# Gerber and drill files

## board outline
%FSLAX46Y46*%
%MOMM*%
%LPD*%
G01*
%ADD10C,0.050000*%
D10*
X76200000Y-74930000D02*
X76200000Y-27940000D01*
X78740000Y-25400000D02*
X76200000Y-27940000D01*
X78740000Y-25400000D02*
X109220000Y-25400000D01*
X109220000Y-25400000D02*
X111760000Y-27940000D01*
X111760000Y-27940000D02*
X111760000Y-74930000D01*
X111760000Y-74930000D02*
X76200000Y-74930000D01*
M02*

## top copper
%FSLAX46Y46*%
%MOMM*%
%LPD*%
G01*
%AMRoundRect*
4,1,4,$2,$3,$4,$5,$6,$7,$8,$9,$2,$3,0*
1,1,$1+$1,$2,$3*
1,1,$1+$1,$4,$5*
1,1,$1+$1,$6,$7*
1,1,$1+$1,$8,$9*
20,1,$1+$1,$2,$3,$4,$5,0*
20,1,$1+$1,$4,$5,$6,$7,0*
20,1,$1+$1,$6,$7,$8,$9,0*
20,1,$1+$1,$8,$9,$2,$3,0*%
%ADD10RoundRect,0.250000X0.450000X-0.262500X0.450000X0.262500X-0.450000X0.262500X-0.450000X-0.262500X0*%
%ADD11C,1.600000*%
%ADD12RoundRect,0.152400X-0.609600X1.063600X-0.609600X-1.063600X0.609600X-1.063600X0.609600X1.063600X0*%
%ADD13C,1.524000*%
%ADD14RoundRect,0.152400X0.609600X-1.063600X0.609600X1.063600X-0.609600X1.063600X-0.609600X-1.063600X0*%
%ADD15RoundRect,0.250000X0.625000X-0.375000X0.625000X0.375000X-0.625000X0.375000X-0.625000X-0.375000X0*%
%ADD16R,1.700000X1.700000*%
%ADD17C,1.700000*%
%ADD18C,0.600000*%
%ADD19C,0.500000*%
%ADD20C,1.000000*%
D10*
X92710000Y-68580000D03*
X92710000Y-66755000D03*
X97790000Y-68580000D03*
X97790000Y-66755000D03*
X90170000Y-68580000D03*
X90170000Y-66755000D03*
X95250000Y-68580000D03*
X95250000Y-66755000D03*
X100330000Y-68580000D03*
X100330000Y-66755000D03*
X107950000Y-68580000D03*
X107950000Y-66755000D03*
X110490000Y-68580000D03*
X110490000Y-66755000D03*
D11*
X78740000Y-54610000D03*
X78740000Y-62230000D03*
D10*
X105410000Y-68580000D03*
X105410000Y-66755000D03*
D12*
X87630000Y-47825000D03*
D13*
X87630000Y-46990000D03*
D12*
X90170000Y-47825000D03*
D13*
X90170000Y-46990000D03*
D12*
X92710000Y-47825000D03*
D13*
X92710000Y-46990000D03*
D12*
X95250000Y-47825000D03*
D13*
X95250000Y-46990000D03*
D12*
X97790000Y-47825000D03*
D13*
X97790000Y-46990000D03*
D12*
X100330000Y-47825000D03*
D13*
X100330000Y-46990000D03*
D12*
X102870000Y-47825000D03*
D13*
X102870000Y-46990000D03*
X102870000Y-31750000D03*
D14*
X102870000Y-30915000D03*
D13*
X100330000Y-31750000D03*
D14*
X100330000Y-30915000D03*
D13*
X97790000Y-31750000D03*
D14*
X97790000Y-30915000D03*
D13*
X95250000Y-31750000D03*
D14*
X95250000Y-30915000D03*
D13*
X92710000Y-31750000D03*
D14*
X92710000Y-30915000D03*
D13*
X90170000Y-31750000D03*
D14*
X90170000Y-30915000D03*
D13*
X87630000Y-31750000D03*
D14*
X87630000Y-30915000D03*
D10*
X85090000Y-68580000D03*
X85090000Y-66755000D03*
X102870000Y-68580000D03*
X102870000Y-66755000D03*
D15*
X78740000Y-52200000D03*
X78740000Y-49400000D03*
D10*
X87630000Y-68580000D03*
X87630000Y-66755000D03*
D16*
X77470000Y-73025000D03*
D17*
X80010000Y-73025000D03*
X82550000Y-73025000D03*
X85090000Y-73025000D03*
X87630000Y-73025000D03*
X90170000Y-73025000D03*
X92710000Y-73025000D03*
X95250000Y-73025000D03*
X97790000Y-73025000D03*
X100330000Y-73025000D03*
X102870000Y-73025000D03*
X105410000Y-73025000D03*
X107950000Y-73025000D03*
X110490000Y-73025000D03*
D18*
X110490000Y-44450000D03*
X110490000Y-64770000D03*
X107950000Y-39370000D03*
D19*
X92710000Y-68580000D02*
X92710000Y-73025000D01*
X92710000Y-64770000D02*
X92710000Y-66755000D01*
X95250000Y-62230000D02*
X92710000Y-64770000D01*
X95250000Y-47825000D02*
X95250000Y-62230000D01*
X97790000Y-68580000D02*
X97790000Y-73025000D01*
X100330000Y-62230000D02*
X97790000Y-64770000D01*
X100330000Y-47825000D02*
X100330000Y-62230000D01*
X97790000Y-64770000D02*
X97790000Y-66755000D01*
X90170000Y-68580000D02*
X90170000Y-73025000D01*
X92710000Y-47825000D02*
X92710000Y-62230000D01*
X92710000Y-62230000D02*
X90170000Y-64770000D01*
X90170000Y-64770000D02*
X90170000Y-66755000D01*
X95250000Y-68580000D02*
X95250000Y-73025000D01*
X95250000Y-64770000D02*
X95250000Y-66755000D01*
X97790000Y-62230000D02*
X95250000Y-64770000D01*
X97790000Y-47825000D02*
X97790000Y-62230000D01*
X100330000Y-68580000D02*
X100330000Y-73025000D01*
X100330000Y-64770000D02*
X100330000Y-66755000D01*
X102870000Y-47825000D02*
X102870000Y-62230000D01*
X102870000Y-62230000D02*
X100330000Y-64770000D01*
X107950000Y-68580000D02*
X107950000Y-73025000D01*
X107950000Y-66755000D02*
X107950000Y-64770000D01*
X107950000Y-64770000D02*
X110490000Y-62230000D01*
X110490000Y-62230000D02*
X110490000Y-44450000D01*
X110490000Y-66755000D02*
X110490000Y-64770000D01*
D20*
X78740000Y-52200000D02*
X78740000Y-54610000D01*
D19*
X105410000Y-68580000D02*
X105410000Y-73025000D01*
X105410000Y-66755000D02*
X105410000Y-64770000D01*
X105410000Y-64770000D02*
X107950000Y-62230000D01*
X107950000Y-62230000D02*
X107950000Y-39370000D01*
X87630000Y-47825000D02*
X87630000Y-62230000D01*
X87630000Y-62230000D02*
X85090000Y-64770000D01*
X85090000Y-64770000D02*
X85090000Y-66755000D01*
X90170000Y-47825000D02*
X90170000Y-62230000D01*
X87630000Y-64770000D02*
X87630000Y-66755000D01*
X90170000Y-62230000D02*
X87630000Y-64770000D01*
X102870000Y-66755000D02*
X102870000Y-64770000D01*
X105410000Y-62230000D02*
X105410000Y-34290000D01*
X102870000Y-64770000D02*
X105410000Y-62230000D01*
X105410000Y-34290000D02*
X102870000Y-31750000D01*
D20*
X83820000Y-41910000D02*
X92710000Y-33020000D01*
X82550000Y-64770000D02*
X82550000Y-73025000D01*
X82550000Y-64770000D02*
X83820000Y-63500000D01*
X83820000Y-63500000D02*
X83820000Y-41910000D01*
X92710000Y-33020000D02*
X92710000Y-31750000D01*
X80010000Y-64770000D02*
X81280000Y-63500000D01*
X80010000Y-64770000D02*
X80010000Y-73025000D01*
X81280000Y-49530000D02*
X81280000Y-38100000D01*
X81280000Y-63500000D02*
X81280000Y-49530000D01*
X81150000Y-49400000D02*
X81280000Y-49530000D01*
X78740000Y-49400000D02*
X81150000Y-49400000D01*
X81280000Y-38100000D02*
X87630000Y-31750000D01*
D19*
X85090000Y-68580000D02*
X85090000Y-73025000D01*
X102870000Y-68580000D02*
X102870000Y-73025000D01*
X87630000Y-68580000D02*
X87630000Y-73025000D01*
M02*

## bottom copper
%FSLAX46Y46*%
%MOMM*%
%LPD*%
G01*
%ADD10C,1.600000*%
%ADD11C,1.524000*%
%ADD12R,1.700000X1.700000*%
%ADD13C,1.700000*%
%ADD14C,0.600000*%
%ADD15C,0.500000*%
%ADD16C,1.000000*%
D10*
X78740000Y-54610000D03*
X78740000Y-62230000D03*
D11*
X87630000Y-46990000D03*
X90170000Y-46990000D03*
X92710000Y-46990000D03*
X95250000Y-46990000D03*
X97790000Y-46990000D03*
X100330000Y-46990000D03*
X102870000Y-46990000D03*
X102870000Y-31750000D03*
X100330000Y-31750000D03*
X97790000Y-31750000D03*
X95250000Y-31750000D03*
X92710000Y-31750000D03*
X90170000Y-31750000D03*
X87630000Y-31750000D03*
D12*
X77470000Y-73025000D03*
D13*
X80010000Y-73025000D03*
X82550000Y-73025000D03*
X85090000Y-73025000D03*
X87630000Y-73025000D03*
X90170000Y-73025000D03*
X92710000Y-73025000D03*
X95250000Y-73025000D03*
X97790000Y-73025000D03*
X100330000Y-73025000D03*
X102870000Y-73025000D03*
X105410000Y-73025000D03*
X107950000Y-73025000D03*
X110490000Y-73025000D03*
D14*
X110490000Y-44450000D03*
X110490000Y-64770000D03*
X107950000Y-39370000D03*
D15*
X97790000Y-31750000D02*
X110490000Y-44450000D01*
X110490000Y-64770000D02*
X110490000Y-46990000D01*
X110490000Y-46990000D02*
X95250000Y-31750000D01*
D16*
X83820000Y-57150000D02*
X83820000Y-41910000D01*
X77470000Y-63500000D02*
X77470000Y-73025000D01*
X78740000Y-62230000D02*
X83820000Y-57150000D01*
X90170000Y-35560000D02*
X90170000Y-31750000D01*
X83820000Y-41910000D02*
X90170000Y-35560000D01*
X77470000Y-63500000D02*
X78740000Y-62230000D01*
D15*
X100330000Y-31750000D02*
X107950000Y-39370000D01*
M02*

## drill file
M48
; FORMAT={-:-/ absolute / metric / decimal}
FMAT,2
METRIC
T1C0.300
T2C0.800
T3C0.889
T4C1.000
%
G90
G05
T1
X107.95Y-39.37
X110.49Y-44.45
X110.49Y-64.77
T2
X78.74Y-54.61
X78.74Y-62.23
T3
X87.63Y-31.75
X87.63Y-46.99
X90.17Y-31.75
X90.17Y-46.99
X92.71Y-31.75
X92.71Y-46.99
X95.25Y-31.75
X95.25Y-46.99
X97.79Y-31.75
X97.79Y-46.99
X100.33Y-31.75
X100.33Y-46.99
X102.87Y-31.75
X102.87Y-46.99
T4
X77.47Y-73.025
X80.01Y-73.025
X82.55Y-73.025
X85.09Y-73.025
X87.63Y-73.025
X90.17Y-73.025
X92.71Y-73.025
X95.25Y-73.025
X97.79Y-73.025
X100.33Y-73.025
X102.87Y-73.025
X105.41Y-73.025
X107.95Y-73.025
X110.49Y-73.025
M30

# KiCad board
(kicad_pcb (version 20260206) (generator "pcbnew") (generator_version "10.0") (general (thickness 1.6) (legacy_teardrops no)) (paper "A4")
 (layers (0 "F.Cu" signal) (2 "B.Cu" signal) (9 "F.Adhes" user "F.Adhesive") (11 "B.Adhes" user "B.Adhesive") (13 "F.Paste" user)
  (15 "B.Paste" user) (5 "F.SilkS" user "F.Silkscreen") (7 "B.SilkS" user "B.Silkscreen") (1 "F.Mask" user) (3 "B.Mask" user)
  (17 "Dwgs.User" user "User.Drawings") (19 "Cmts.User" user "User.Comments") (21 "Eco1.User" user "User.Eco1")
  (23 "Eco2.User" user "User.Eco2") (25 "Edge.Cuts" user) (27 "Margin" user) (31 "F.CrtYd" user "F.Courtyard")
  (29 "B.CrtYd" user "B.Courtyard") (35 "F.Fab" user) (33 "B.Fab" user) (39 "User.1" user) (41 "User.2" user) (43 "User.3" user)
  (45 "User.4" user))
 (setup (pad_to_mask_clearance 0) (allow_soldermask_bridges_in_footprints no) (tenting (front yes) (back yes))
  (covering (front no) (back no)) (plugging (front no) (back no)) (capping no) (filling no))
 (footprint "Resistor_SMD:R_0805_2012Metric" (layer "F.Cu") (at 92.71 67.6675 90)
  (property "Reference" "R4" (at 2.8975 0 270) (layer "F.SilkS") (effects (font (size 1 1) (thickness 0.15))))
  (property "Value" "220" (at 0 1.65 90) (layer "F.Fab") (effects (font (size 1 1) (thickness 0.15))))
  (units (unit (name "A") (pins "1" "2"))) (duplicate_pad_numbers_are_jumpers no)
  (pad "1" smd roundrect (at -0.9125 0 90) (size 1.025 1.4) (layers "F.Cu" "F.Mask" "F.Paste") (roundrect_rratio 0.243902)
   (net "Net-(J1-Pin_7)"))
  (pad "2" smd roundrect (at 0.9125 0 90) (size 1.025 1.4) (layers "F.Cu" "F.Mask" "F.Paste") (roundrect_rratio 0.243902) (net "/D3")))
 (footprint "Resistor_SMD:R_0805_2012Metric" (layer "F.Cu") (at 97.79 67.6675 90)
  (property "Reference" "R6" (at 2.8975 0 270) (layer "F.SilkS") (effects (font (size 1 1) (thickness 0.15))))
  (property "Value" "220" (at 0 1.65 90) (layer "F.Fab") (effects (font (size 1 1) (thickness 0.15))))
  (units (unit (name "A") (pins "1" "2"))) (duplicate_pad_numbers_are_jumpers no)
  (pad "1" smd roundrect (at -0.9125 0 90) (size 1.025 1.4) (layers "F.Cu" "F.Mask" "F.Paste") (roundrect_rratio 0.243902)
   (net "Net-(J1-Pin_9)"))
  (pad "2" smd roundrect (at 0.9125 0 90) (size 1.025 1.4) (layers "F.Cu" "F.Mask" "F.Paste") (roundrect_rratio 0.243902) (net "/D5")))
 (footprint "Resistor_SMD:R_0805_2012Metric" (layer "F.Cu") (at 90.17 67.6675 90)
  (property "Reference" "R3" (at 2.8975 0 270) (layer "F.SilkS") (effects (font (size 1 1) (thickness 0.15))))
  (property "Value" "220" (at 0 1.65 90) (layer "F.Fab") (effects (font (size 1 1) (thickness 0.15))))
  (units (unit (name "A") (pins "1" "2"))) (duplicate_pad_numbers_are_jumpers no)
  (pad "1" smd roundrect (at -0.9125 0 90) (size 1.025 1.4) (layers "F.Cu" "F.Mask" "F.Paste") (roundrect_rratio 0.243902)
   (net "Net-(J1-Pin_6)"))
  (pad "2" smd roundrect (at 0.9125 0 90) (size 1.025 1.4) (layers "F.Cu" "F.Mask" "F.Paste") (roundrect_rratio 0.243902) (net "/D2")))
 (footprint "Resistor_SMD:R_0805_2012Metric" (layer "F.Cu") (at 95.25 67.6675 90)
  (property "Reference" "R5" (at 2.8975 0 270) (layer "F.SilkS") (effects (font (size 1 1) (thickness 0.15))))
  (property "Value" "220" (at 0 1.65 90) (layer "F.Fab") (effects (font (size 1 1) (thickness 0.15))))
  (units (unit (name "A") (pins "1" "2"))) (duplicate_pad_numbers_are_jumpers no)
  (pad "1" smd roundrect (at -0.9125 0 90) (size 1.025 1.4) (layers "F.Cu" "F.Mask" "F.Paste") (roundrect_rratio 0.243902)
   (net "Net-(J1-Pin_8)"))
  (pad "2" smd roundrect (at 0.9125 0 90) (size 1.025 1.4) (layers "F.Cu" "F.Mask" "F.Paste") (roundrect_rratio 0.243902) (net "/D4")))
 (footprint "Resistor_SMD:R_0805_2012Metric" (layer "F.Cu") (at 100.33 67.6675 90)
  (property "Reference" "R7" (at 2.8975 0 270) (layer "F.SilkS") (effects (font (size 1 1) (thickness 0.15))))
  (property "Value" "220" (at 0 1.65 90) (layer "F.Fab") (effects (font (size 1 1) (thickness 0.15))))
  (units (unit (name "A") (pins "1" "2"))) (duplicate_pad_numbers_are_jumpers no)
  (pad "1" smd roundrect (at -0.9125 0 90) (size 1.025 1.4) (layers "F.Cu" "F.Mask" "F.Paste") (roundrect_rratio 0.243902)
   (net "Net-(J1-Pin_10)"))
  (pad "2" smd roundrect (at 0.9125 0 90) (size 1.025 1.4) (layers "F.Cu" "F.Mask" "F.Paste") (roundrect_rratio 0.243902) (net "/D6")))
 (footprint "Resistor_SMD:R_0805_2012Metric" (layer "F.Cu") (at 107.95 67.6675 90)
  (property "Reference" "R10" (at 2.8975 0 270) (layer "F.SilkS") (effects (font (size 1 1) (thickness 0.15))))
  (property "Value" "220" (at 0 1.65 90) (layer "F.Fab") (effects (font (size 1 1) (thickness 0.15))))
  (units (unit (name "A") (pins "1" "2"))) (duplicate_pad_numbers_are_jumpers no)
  (pad "1" smd roundrect (at -0.9125 0 90) (size 1.025 1.4) (layers "F.Cu" "F.Mask" "F.Paste") (roundrect_rratio 0.243902)
   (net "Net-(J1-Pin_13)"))
  (pad "2" smd roundrect (at 0.9125 0 90) (size 1.025 1.4) (layers "F.Cu" "F.Mask" "F.Paste") (roundrect_rratio 0.243902) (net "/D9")))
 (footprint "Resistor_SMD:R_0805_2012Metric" (layer "F.Cu") (at 110.49 67.6675 90)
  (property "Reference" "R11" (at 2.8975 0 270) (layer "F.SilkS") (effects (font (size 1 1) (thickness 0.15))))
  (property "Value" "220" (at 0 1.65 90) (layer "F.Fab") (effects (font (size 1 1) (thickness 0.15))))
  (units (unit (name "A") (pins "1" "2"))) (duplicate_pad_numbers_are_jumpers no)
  (pad "1" smd roundrect (at -0.9125 0 90) (size 1.025 1.4) (layers "F.Cu" "F.Mask" "F.Paste") (roundrect_rratio 0.243902)
   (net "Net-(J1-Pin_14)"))
  (pad "2" smd roundrect (at 0.9125 0 90) (size 1.025 1.4) (layers "F.Cu" "F.Mask" "F.Paste") (roundrect_rratio 0.243902) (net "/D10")))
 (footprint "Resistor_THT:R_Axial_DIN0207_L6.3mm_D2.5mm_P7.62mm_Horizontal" (layer "F.Cu") (at 78.74 54.61 -90)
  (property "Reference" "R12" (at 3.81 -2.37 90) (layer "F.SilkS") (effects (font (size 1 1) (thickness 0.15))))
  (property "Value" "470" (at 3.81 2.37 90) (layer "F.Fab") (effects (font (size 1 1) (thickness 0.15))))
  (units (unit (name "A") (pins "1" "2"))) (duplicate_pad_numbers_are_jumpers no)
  (pad "1" thru_hole circle (at 0 0 270) (size 1.6 1.6) (drill 0.8) (layers "*.Cu" "*.Mask") (remove_unused_layers no) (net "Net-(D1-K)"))
  (pad "2" thru_hole circle (at 7.62 0 270) (size 1.6 1.6) (drill 0.8) (layers "*.Cu" "*.Mask") (remove_unused_layers no) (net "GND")))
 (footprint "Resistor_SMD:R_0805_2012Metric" (layer "F.Cu") (at 105.41 67.6675 90)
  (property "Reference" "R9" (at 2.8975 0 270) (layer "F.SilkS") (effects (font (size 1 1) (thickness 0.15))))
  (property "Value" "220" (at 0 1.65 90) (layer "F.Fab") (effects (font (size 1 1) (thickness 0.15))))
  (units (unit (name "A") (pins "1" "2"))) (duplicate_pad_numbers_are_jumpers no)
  (pad "1" smd roundrect (at -0.9125 0 90) (size 1.025 1.4) (layers "F.Cu" "F.Mask" "F.Paste") (roundrect_rratio 0.243902)
   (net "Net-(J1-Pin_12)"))
  (pad "2" smd roundrect (at 0.9125 0 90) (size 1.025 1.4) (layers "F.Cu" "F.Mask" "F.Paste") (roundrect_rratio 0.243902) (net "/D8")))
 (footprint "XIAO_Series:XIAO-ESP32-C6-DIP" (layer "F.Cu") (at 95.25 39.37 180)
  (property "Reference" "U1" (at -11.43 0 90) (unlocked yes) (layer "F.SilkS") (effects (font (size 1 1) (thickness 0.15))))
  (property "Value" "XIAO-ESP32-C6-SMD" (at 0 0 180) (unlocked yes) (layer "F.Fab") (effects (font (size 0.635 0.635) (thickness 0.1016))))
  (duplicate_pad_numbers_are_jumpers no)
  (pad "1" smd roundrect (at 7.62 -8.455 270) (size 2.432 1.524) (layers "F.Cu" "F.Mask") (roundrect_rratio 0.1) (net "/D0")
   (thermal_bridge_angle 45))
  (pad "1" thru_hole circle (at 7.62 -7.62 270) (size 1.524 1.524) (drill 0.889) (layers "*.Cu" "*.Mask") (remove_unused_layers no)
   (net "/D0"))
  (pad "2" smd roundrect (at 5.08 -8.455 270) (size 2.432 1.524) (layers "F.Cu" "F.Mask") (roundrect_rratio 0.1) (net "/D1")
   (thermal_bridge_angle 45))
  (pad "2" thru_hole circle (at 5.08 -7.62 270) (size 1.524 1.524) (drill 0.889) (layers "*.Cu" "*.Mask") (remove_unused_layers no)
   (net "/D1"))
  (pad "3" smd roundrect (at 2.54 -8.455 270) (size 2.432 1.524) (layers "F.Cu" "F.Mask") (roundrect_rratio 0.1) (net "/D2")
   (thermal_bridge_angle 45))
  (pad "3" thru_hole circle (at 2.54 -7.62 270) (size 1.524 1.524) (drill 0.889) (layers "*.Cu" "*.Mask") (remove_unused_layers no)
   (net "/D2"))
  (pad "4" smd roundrect (at 0 -8.455 270) (size 2.432 1.524) (layers "F.Cu" "F.Mask") (roundrect_rratio 0.1) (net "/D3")
   (thermal_bridge_angle 45))
  (pad "4" thru_hole circle (at 0 -7.62 270) (size 1.524 1.524) (drill 0.889) (layers "*.Cu" "*.Mask") (remove_unused_layers no) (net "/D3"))
  (pad "5" smd roundrect (at -2.54 -8.455 270) (size 2.432 1.524) (layers "F.Cu" "F.Mask") (roundrect_rratio 0.1) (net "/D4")
   (thermal_bridge_angle 45))
  (pad "5" thru_hole circle (at -2.54 -7.62 270) (size 1.524 1.524) (drill 0.889) (layers "*.Cu" "*.Mask") (remove_unused_layers no)
   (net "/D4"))
  (pad "6" smd roundrect (at -5.08 -8.455 270) (size 2.432 1.524) (layers "F.Cu" "F.Mask") (roundrect_rratio 0.1) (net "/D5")
   (thermal_bridge_angle 45))
  (pad "6" thru_hole circle (at -5.08 -7.62 270) (size 1.524 1.524) (drill 0.889) (layers "*.Cu" "*.Mask") (remove_unused_layers no)
   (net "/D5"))
  (pad "7" smd roundrect (at -7.62 -8.455 270) (size 2.432 1.524) (layers "F.Cu" "F.Mask") (roundrect_rratio 0.1) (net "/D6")
   (thermal_bridge_angle 45))
  (pad "7" thru_hole circle (at -7.62 -7.62 270) (size 1.524 1.524) (drill 0.889) (layers "*.Cu" "*.Mask") (remove_unused_layers no)
   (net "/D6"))
  (pad "8" thru_hole circle (at -7.62 7.62 90) (size 1.524 1.524) (drill 0.889) (layers "*.Cu" "*.Mask") (remove_unused_layers no)
   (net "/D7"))
  (pad "8" smd roundrect (at -7.62 8.455 90) (size 2.432 1.524) (layers "F.Cu" "F.Mask") (roundrect_rratio 0.1) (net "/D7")
   (thermal_bridge_angle 45))
  (pad "9" thru_hole circle (at -5.08 7.62 90) (size 1.524 1.524) (drill 0.889) (layers "*.Cu" "*.Mask") (remove_unused_layers no)
   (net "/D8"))
  (pad "9" smd roundrect (at -5.08 8.455 90) (size 2.432 1.524) (layers "F.Cu" "F.Mask") (roundrect_rratio 0.1) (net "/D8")
   (thermal_bridge_angle 45))
  (pad "10" thru_hole circle (at -2.54 7.62 90) (size 1.524 1.524) (drill 0.889) (layers "*.Cu" "*.Mask") (remove_unused_layers no)
   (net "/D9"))
  (pad "10" smd roundrect (at -2.54 8.455 90) (size 2.432 1.524) (layers "F.Cu" "F.Mask") (roundrect_rratio 0.1) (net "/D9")
   (thermal_bridge_angle 45))
  (pad "11" thru_hole circle (at 0 7.62 90) (size 1.524 1.524) (drill 0.889) (layers "*.Cu" "*.Mask") (remove_unused_layers no) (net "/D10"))
  (pad "11" smd roundrect (at 0 8.455 90) (size 2.432 1.524) (layers "F.Cu" "F.Mask") (roundrect_rratio 0.1) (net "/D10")
   (thermal_bridge_angle 45))
  (pad "12" thru_hole circle (at 2.54 7.62 90) (size 1.524 1.524) (drill 0.889) (layers "*.Cu" "*.Mask") (remove_unused_layers no)
   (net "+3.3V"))
  (pad "12" smd roundrect (at 2.54 8.455 90) (size 2.432 1.524) (layers "F.Cu" "F.Mask") (roundrect_rratio 0.1) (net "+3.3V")
   (thermal_bridge_angle 45))
  (pad "13" thru_hole circle (at 5.08 7.62 90) (size 1.524 1.524) (drill 0.889) (layers "*.Cu" "*.Mask") (remove_unused_layers no)
   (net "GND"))
  (pad "13" smd roundrect (at 5.08 8.455 90) (size 2.432 1.524) (layers "F.Cu" "F.Mask") (roundrect_rratio 0.1) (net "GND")
   (thermal_bridge_angle 45))
  (pad "14" thru_hole circle (at 7.62 7.62 90) (size 1.524 1.524) (drill 0.889) (layers "*.Cu" "*.Mask") (remove_unused_layers no)
   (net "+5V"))
  (pad "14" smd roundrect (at 7.62 8.455 90) (size 2.432 1.524) (layers "F.Cu" "F.Mask") (roundrect_rratio 0.1) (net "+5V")
   (thermal_bridge_angle 45)))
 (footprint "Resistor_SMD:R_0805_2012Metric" (layer "F.Cu") (at 85.09 67.6675 90)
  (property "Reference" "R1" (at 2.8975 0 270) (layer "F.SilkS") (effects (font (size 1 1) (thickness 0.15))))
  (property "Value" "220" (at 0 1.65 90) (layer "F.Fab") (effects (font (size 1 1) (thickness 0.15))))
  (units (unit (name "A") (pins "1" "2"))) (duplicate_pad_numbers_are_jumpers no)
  (pad "1" smd roundrect (at -0.9125 0 90) (size 1.025 1.4) (layers "F.Cu" "F.Mask" "F.Paste") (roundrect_rratio 0.243902)
   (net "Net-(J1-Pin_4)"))
  (pad "2" smd roundrect (at 0.9125 0 90) (size 1.025 1.4) (layers "F.Cu" "F.Mask" "F.Paste") (roundrect_rratio 0.243902) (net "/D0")))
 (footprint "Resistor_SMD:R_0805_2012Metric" (layer "F.Cu") (at 102.87 67.6675 90)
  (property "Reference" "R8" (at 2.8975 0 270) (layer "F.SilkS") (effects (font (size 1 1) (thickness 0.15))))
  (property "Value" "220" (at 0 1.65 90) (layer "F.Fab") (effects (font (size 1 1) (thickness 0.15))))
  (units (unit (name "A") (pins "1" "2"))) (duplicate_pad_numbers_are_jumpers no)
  (pad "1" smd roundrect (at -0.9125 0 90) (size 1.025 1.4) (layers "F.Cu" "F.Mask" "F.Paste") (roundrect_rratio 0.243902)
   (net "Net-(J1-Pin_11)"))
  (pad "2" smd roundrect (at 0.9125 0 90) (size 1.025 1.4) (layers "F.Cu" "F.Mask" "F.Paste") (roundrect_rratio 0.243902) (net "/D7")))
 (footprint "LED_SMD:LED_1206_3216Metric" (layer "F.Cu") (at 78.74 50.8 90)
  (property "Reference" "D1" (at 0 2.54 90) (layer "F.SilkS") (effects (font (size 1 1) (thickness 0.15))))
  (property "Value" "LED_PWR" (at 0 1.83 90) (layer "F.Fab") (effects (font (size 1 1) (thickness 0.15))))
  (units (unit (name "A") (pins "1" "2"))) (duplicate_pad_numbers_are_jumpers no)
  (pad "1" smd roundrect (at -1.4 0 90) (size 1.25 1.75) (layers "F.Cu" "F.Mask" "F.Paste") (roundrect_rratio 0.2) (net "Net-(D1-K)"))
  (pad "2" smd roundrect (at 1.4 0 90) (size 1.25 1.75) (layers "F.Cu" "F.Mask" "F.Paste") (roundrect_rratio 0.2) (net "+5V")))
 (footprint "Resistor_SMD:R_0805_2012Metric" (layer "F.Cu") (at 87.63 67.6675 90)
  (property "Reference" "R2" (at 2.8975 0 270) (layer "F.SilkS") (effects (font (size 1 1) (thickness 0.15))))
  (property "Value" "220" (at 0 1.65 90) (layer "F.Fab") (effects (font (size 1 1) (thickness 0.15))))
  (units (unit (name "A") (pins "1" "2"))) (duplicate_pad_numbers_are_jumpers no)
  (pad "1" smd roundrect (at -0.9125 0 90) (size 1.025 1.4) (layers "F.Cu" "F.Mask" "F.Paste") (roundrect_rratio 0.243902)
   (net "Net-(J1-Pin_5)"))
  (pad "2" smd roundrect (at 0.9125 0 90) (size 1.025 1.4) (layers "F.Cu" "F.Mask" "F.Paste") (roundrect_rratio 0.243902) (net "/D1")))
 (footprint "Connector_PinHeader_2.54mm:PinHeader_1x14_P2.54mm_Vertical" (layer "F.Cu") (at 77.47 73.025 90)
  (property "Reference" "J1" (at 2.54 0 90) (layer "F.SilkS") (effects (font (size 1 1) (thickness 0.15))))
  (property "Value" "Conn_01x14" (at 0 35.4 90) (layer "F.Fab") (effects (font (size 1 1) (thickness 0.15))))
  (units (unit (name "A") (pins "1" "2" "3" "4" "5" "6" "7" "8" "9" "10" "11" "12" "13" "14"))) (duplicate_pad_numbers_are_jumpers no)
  (pad "1" thru_hole rect (at 0 0 90) (size 1.7 1.7) (drill 1) (layers "*.Cu" "*.Mask") (remove_unused_layers no) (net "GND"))
  (pad "2" thru_hole circle (at 0 2.54 90) (size 1.7 1.7) (drill 1) (layers "*.Cu" "*.Mask") (remove_unused_layers no) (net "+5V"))
  (pad "3" thru_hole circle (at 0 5.08 90) (size 1.7 1.7) (drill 1) (layers "*.Cu" "*.Mask") (remove_unused_layers no) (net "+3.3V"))
  (pad "4" thru_hole circle (at 0 7.62 90) (size 1.7 1.7) (drill 1) (layers "*.Cu" "*.Mask") (remove_unused_layers no)
   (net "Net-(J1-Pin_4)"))
  (pad "5" thru_hole circle (at 0 10.16 90) (size 1.7 1.7) (drill 1) (layers "*.Cu" "*.Mask") (remove_unused_layers no)
   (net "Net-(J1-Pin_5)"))
  (pad "6" thru_hole circle (at 0 12.7 90) (size 1.7 1.7) (drill 1) (layers "*.Cu" "*.Mask") (remove_unused_layers no)
   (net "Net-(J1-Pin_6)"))
  (pad "7" thru_hole circle (at 0 15.24 90) (size 1.7 1.7) (drill 1) (layers "*.Cu" "*.Mask") (remove_unused_layers no)
   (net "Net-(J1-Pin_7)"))
  (pad "8" thru_hole circle (at 0 17.78 90) (size 1.7 1.7) (drill 1) (layers "*.Cu" "*.Mask") (remove_unused_layers no)
   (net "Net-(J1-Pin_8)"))
  (pad "9" thru_hole circle (at 0 20.32 90) (size 1.7 1.7) (drill 1) (layers "*.Cu" "*.Mask") (remove_unused_layers no)
   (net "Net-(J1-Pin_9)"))
  (pad "10" thru_hole circle (at 0 22.86 90) (size 1.7 1.7) (drill 1) (layers "*.Cu" "*.Mask") (remove_unused_layers no)
   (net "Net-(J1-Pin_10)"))
  (pad "11" thru_hole circle (at 0 25.4 90) (size 1.7 1.7) (drill 1) (layers "*.Cu" "*.Mask") (remove_unused_layers no)
   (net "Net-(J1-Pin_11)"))
  (pad "12" thru_hole circle (at 0 27.94 90) (size 1.7 1.7) (drill 1) (layers "*.Cu" "*.Mask") (remove_unused_layers no)
   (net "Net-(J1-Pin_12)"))
  (pad "13" thru_hole circle (at 0 30.48 90) (size 1.7 1.7) (drill 1) (layers "*.Cu" "*.Mask") (remove_unused_layers no)
   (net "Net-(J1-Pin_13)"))
  (pad "14" thru_hole circle (at 0 33.02 90) (size 1.7 1.7) (drill 1) (layers "*.Cu" "*.Mask") (remove_unused_layers no)
   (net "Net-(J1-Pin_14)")))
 (gr_line (start 76.2 74.93) (end 76.2 27.94) (stroke (width 0.05) (type default)) (layer "Edge.Cuts"))
 (gr_line (start 78.74 25.4) (end 76.2 27.94) (stroke (width 0.05) (type default)) (layer "Edge.Cuts"))
 (gr_line (start 78.74 25.4) (end 109.22 25.4) (stroke (width 0.05) (type default)) (layer "Edge.Cuts"))
 (gr_line (start 109.22 25.4) (end 111.76 27.94) (stroke (width 0.05) (type default)) (layer "Edge.Cuts"))
 (gr_line (start 111.76 27.94) (end 111.76 74.93) (stroke (width 0.05) (type default)) (layer "Edge.Cuts"))
 (gr_line (start 111.76 74.93) (end 76.2 74.93) (stroke (width 0.05) (type default)) (layer "Edge.Cuts"))
 (segment (start 92.71 68.58) (end 92.71 73.025) (width 0.5) (layer "F.Cu") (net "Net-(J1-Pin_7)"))
 (segment (start 92.71 64.77) (end 92.71 66.755) (width 0.5) (layer "F.Cu") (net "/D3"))
 (segment (start 95.25 62.23) (end 92.71 64.77) (width 0.5) (layer "F.Cu") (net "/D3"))
 (segment (start 95.25 47.825) (end 95.25 62.23) (width 0.5) (layer "F.Cu") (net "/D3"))
 (segment (start 97.79 68.58) (end 97.79 73.025) (width 0.5) (layer "F.Cu") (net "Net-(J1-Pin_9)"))
 (segment (start 100.33 62.23) (end 97.79 64.77) (width 0.5) (layer "F.Cu") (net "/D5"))
 (segment (start 100.33 47.825) (end 100.33 62.23) (width 0.5) (layer "F.Cu") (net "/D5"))
 (segment (start 97.79 64.77) (end 97.79 66.755) (width 0.5) (layer "F.Cu") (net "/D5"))
 (segment (start 90.17 68.58) (end 90.17 73.025) (width 0.5) (layer "F.Cu") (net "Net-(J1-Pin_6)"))
 (segment (start 92.71 47.825) (end 92.71 62.23) (width 0.5) (layer "F.Cu") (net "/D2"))
 (segment (start 92.71 62.23) (end 90.17 64.77) (width 0.5) (layer "F.Cu") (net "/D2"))
 (segment (start 90.17 64.77) (end 90.17 66.755) (width 0.5) (layer "F.Cu") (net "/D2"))
 (segment (start 95.25 68.58) (end 95.25 73.025) (width 0.5) (layer "F.Cu") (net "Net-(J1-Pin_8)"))
 (segment (start 95.25 64.77) (end 95.25 66.755) (width 0.5) (layer "F.Cu") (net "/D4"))
 (segment (start 97.79 62.23) (end 95.25 64.77) (width 0.5) (layer "F.Cu") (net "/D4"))
 (segment (start 97.79 47.825) (end 97.79 62.23) (width 0.5) (layer "F.Cu") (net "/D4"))
 (segment (start 100.33 68.58) (end 100.33 73.025) (width 0.5) (layer "F.Cu") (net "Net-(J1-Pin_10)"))
 (segment (start 100.33 64.77) (end 100.33 66.755) (width 0.5) (layer "F.Cu") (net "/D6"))
 (segment (start 102.87 47.825) (end 102.87 62.23) (width 0.5) (layer "F.Cu") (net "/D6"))
 (segment (start 102.87 62.23) (end 100.33 64.77) (width 0.5) (layer "F.Cu") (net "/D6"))
 (segment (start 107.95 68.58) (end 107.95 73.025) (width 0.5) (layer "F.Cu") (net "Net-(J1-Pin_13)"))
 (segment (start 107.95 66.755) (end 107.95 64.77) (width 0.5) (layer "F.Cu") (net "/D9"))
 (segment (start 107.95 64.77) (end 110.49 62.23) (width 0.5) (layer "F.Cu") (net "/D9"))
 (segment (start 110.49 62.23) (end 110.49 44.45) (width 0.5) (layer "F.Cu") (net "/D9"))
 (via (at 110.49 44.45) (size 0.6) (drill 0.3) (layers "F.Cu" "B.Cu") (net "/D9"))
 (segment (start 97.79 31.75) (end 110.49 44.45) (width 0.5) (layer "B.Cu") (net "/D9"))
 (segment (start 110.49 66.755) (end 110.49 64.77) (width 0.5) (layer "F.Cu") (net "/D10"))
 (via (at 110.49 64.77) (size 0.6) (drill 0.3) (layers "F.Cu" "B.Cu") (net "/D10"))
 (segment (start 110.49 64.77) (end 110.49 46.99) (width 0.5) (layer "B.Cu") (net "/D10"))
 (segment (start 110.49 46.99) (end 95.25 31.75) (width 0.5) (layer "B.Cu") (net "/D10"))
 (segment (start 78.74 52.2) (end 78.74 54.61) (width 1) (layer "F.Cu") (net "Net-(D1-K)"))
 (segment (start 83.82 57.15) (end 83.82 41.91) (width 1) (layer "B.Cu") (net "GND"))
 (segment (start 77.47 63.5) (end 77.47 73.025) (width 1) (layer "B.Cu") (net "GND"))
 (segment (start 78.74 62.23) (end 83.82 57.15) (width 1) (layer "B.Cu") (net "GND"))
 (segment (start 90.17 35.56) (end 90.17 31.75) (width 1) (layer "B.Cu") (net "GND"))
 (segment (start 83.82 41.91) (end 90.17 35.56) (width 1) (layer "B.Cu") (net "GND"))
 (segment (start 77.47 63.5) (end 78.74 62.23) (width 1) (layer "B.Cu") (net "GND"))
 (segment (start 105.41 68.58) (end 105.41 73.025) (width 0.5) (layer "F.Cu") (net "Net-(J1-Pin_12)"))
 (segment (start 105.41 66.755) (end 105.41 64.77) (width 0.5) (layer "F.Cu") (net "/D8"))
 (segment (start 105.41 64.77) (end 107.95 62.23) (width 0.5) (layer "F.Cu") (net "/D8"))
 (segment (start 107.95 62.23) (end 107.95 39.37) (width 0.5) (layer "F.Cu") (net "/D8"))
 (via (at 107.95 39.37) (size 0.6) (drill 0.3) (layers "F.Cu" "B.Cu") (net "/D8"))
 (segment (start 100.33 31.75) (end 107.95 39.37) (width 0.5) (layer "B.Cu") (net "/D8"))
 (segment (start 87.63 47.825) (end 87.63 62.23) (width 0.5) (layer "F.Cu") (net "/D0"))
 (segment (start 87.63 62.23) (end 85.09 64.77) (width 0.5) (layer "F.Cu") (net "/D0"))
 (segment (start 85.09 64.77) (end 85.09 66.755) (width 0.5) (layer "F.Cu") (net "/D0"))
 (segment (start 90.17 47.825) (end 90.17 62.23) (width 0.5) (layer "F.Cu") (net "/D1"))
 (segment (start 87.63 64.77) (end 87.63 66.755) (width 0.5) (layer "F.Cu") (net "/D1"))
 (segment (start 90.17 62.23) (end 87.63 64.77) (width 0.5) (layer "F.Cu") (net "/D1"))
 (segment (start 102.87 66.755) (end 102.87 64.77) (width 0.5) (layer "F.Cu") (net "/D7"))
 (segment (start 105.41 62.23) (end 105.41 34.29) (width 0.5) (layer "F.Cu") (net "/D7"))
 (segment (start 102.87 64.77) (end 105.41 62.23) (width 0.5) (layer "F.Cu") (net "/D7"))
 (segment (start 105.41 34.29) (end 102.87 31.75) (width 0.5) (layer "F.Cu") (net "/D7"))
 (segment (start 83.82 41.91) (end 92.71 33.02) (width 1) (layer "F.Cu") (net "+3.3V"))
 (segment (start 82.55 64.77) (end 82.55 73.025) (width 1) (layer "F.Cu") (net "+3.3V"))
 (segment (start 82.55 64.77) (end 83.82 63.5) (width 1) (layer "F.Cu") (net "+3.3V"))
 (segment (start 83.82 63.5) (end 83.82 41.91) (width 1) (layer "F.Cu") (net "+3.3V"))
 (segment (start 92.71 33.02) (end 92.71 31.75) (width 1) (layer "F.Cu") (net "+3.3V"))
 (segment (start 80.01 64.77) (end 81.28 63.5) (width 1) (layer "F.Cu") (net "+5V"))
 (segment (start 80.01 64.77) (end 80.01 73.025) (width 1) (layer "F.Cu") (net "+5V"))
 (segment (start 81.28 49.53) (end 81.28 38.1) (width 1) (layer "F.Cu") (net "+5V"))
 (segment (start 81.28 63.5) (end 81.28 49.53) (width 1) (layer "F.Cu") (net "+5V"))
 (segment (start 81.15 49.4) (end 81.28 49.53) (width 1) (layer "F.Cu") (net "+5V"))
 (segment (start 78.74 49.4) (end 81.15 49.4) (width 1) (layer "F.Cu") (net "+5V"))
 (segment (start 81.28 38.1) (end 87.63 31.75) (width 1) (layer "F.Cu") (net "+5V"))
 (segment (start 85.09 68.58) (end 85.09 73.025) (width 0.5) (layer "F.Cu") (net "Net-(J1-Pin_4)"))
 (segment (start 102.87 68.58) (end 102.87 73.025) (width 0.5) (layer "F.Cu") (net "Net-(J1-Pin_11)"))
 (segment (start 87.63 68.58) (end 87.63 73.025) (width 0.5) (layer "F.Cu") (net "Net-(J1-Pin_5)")))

